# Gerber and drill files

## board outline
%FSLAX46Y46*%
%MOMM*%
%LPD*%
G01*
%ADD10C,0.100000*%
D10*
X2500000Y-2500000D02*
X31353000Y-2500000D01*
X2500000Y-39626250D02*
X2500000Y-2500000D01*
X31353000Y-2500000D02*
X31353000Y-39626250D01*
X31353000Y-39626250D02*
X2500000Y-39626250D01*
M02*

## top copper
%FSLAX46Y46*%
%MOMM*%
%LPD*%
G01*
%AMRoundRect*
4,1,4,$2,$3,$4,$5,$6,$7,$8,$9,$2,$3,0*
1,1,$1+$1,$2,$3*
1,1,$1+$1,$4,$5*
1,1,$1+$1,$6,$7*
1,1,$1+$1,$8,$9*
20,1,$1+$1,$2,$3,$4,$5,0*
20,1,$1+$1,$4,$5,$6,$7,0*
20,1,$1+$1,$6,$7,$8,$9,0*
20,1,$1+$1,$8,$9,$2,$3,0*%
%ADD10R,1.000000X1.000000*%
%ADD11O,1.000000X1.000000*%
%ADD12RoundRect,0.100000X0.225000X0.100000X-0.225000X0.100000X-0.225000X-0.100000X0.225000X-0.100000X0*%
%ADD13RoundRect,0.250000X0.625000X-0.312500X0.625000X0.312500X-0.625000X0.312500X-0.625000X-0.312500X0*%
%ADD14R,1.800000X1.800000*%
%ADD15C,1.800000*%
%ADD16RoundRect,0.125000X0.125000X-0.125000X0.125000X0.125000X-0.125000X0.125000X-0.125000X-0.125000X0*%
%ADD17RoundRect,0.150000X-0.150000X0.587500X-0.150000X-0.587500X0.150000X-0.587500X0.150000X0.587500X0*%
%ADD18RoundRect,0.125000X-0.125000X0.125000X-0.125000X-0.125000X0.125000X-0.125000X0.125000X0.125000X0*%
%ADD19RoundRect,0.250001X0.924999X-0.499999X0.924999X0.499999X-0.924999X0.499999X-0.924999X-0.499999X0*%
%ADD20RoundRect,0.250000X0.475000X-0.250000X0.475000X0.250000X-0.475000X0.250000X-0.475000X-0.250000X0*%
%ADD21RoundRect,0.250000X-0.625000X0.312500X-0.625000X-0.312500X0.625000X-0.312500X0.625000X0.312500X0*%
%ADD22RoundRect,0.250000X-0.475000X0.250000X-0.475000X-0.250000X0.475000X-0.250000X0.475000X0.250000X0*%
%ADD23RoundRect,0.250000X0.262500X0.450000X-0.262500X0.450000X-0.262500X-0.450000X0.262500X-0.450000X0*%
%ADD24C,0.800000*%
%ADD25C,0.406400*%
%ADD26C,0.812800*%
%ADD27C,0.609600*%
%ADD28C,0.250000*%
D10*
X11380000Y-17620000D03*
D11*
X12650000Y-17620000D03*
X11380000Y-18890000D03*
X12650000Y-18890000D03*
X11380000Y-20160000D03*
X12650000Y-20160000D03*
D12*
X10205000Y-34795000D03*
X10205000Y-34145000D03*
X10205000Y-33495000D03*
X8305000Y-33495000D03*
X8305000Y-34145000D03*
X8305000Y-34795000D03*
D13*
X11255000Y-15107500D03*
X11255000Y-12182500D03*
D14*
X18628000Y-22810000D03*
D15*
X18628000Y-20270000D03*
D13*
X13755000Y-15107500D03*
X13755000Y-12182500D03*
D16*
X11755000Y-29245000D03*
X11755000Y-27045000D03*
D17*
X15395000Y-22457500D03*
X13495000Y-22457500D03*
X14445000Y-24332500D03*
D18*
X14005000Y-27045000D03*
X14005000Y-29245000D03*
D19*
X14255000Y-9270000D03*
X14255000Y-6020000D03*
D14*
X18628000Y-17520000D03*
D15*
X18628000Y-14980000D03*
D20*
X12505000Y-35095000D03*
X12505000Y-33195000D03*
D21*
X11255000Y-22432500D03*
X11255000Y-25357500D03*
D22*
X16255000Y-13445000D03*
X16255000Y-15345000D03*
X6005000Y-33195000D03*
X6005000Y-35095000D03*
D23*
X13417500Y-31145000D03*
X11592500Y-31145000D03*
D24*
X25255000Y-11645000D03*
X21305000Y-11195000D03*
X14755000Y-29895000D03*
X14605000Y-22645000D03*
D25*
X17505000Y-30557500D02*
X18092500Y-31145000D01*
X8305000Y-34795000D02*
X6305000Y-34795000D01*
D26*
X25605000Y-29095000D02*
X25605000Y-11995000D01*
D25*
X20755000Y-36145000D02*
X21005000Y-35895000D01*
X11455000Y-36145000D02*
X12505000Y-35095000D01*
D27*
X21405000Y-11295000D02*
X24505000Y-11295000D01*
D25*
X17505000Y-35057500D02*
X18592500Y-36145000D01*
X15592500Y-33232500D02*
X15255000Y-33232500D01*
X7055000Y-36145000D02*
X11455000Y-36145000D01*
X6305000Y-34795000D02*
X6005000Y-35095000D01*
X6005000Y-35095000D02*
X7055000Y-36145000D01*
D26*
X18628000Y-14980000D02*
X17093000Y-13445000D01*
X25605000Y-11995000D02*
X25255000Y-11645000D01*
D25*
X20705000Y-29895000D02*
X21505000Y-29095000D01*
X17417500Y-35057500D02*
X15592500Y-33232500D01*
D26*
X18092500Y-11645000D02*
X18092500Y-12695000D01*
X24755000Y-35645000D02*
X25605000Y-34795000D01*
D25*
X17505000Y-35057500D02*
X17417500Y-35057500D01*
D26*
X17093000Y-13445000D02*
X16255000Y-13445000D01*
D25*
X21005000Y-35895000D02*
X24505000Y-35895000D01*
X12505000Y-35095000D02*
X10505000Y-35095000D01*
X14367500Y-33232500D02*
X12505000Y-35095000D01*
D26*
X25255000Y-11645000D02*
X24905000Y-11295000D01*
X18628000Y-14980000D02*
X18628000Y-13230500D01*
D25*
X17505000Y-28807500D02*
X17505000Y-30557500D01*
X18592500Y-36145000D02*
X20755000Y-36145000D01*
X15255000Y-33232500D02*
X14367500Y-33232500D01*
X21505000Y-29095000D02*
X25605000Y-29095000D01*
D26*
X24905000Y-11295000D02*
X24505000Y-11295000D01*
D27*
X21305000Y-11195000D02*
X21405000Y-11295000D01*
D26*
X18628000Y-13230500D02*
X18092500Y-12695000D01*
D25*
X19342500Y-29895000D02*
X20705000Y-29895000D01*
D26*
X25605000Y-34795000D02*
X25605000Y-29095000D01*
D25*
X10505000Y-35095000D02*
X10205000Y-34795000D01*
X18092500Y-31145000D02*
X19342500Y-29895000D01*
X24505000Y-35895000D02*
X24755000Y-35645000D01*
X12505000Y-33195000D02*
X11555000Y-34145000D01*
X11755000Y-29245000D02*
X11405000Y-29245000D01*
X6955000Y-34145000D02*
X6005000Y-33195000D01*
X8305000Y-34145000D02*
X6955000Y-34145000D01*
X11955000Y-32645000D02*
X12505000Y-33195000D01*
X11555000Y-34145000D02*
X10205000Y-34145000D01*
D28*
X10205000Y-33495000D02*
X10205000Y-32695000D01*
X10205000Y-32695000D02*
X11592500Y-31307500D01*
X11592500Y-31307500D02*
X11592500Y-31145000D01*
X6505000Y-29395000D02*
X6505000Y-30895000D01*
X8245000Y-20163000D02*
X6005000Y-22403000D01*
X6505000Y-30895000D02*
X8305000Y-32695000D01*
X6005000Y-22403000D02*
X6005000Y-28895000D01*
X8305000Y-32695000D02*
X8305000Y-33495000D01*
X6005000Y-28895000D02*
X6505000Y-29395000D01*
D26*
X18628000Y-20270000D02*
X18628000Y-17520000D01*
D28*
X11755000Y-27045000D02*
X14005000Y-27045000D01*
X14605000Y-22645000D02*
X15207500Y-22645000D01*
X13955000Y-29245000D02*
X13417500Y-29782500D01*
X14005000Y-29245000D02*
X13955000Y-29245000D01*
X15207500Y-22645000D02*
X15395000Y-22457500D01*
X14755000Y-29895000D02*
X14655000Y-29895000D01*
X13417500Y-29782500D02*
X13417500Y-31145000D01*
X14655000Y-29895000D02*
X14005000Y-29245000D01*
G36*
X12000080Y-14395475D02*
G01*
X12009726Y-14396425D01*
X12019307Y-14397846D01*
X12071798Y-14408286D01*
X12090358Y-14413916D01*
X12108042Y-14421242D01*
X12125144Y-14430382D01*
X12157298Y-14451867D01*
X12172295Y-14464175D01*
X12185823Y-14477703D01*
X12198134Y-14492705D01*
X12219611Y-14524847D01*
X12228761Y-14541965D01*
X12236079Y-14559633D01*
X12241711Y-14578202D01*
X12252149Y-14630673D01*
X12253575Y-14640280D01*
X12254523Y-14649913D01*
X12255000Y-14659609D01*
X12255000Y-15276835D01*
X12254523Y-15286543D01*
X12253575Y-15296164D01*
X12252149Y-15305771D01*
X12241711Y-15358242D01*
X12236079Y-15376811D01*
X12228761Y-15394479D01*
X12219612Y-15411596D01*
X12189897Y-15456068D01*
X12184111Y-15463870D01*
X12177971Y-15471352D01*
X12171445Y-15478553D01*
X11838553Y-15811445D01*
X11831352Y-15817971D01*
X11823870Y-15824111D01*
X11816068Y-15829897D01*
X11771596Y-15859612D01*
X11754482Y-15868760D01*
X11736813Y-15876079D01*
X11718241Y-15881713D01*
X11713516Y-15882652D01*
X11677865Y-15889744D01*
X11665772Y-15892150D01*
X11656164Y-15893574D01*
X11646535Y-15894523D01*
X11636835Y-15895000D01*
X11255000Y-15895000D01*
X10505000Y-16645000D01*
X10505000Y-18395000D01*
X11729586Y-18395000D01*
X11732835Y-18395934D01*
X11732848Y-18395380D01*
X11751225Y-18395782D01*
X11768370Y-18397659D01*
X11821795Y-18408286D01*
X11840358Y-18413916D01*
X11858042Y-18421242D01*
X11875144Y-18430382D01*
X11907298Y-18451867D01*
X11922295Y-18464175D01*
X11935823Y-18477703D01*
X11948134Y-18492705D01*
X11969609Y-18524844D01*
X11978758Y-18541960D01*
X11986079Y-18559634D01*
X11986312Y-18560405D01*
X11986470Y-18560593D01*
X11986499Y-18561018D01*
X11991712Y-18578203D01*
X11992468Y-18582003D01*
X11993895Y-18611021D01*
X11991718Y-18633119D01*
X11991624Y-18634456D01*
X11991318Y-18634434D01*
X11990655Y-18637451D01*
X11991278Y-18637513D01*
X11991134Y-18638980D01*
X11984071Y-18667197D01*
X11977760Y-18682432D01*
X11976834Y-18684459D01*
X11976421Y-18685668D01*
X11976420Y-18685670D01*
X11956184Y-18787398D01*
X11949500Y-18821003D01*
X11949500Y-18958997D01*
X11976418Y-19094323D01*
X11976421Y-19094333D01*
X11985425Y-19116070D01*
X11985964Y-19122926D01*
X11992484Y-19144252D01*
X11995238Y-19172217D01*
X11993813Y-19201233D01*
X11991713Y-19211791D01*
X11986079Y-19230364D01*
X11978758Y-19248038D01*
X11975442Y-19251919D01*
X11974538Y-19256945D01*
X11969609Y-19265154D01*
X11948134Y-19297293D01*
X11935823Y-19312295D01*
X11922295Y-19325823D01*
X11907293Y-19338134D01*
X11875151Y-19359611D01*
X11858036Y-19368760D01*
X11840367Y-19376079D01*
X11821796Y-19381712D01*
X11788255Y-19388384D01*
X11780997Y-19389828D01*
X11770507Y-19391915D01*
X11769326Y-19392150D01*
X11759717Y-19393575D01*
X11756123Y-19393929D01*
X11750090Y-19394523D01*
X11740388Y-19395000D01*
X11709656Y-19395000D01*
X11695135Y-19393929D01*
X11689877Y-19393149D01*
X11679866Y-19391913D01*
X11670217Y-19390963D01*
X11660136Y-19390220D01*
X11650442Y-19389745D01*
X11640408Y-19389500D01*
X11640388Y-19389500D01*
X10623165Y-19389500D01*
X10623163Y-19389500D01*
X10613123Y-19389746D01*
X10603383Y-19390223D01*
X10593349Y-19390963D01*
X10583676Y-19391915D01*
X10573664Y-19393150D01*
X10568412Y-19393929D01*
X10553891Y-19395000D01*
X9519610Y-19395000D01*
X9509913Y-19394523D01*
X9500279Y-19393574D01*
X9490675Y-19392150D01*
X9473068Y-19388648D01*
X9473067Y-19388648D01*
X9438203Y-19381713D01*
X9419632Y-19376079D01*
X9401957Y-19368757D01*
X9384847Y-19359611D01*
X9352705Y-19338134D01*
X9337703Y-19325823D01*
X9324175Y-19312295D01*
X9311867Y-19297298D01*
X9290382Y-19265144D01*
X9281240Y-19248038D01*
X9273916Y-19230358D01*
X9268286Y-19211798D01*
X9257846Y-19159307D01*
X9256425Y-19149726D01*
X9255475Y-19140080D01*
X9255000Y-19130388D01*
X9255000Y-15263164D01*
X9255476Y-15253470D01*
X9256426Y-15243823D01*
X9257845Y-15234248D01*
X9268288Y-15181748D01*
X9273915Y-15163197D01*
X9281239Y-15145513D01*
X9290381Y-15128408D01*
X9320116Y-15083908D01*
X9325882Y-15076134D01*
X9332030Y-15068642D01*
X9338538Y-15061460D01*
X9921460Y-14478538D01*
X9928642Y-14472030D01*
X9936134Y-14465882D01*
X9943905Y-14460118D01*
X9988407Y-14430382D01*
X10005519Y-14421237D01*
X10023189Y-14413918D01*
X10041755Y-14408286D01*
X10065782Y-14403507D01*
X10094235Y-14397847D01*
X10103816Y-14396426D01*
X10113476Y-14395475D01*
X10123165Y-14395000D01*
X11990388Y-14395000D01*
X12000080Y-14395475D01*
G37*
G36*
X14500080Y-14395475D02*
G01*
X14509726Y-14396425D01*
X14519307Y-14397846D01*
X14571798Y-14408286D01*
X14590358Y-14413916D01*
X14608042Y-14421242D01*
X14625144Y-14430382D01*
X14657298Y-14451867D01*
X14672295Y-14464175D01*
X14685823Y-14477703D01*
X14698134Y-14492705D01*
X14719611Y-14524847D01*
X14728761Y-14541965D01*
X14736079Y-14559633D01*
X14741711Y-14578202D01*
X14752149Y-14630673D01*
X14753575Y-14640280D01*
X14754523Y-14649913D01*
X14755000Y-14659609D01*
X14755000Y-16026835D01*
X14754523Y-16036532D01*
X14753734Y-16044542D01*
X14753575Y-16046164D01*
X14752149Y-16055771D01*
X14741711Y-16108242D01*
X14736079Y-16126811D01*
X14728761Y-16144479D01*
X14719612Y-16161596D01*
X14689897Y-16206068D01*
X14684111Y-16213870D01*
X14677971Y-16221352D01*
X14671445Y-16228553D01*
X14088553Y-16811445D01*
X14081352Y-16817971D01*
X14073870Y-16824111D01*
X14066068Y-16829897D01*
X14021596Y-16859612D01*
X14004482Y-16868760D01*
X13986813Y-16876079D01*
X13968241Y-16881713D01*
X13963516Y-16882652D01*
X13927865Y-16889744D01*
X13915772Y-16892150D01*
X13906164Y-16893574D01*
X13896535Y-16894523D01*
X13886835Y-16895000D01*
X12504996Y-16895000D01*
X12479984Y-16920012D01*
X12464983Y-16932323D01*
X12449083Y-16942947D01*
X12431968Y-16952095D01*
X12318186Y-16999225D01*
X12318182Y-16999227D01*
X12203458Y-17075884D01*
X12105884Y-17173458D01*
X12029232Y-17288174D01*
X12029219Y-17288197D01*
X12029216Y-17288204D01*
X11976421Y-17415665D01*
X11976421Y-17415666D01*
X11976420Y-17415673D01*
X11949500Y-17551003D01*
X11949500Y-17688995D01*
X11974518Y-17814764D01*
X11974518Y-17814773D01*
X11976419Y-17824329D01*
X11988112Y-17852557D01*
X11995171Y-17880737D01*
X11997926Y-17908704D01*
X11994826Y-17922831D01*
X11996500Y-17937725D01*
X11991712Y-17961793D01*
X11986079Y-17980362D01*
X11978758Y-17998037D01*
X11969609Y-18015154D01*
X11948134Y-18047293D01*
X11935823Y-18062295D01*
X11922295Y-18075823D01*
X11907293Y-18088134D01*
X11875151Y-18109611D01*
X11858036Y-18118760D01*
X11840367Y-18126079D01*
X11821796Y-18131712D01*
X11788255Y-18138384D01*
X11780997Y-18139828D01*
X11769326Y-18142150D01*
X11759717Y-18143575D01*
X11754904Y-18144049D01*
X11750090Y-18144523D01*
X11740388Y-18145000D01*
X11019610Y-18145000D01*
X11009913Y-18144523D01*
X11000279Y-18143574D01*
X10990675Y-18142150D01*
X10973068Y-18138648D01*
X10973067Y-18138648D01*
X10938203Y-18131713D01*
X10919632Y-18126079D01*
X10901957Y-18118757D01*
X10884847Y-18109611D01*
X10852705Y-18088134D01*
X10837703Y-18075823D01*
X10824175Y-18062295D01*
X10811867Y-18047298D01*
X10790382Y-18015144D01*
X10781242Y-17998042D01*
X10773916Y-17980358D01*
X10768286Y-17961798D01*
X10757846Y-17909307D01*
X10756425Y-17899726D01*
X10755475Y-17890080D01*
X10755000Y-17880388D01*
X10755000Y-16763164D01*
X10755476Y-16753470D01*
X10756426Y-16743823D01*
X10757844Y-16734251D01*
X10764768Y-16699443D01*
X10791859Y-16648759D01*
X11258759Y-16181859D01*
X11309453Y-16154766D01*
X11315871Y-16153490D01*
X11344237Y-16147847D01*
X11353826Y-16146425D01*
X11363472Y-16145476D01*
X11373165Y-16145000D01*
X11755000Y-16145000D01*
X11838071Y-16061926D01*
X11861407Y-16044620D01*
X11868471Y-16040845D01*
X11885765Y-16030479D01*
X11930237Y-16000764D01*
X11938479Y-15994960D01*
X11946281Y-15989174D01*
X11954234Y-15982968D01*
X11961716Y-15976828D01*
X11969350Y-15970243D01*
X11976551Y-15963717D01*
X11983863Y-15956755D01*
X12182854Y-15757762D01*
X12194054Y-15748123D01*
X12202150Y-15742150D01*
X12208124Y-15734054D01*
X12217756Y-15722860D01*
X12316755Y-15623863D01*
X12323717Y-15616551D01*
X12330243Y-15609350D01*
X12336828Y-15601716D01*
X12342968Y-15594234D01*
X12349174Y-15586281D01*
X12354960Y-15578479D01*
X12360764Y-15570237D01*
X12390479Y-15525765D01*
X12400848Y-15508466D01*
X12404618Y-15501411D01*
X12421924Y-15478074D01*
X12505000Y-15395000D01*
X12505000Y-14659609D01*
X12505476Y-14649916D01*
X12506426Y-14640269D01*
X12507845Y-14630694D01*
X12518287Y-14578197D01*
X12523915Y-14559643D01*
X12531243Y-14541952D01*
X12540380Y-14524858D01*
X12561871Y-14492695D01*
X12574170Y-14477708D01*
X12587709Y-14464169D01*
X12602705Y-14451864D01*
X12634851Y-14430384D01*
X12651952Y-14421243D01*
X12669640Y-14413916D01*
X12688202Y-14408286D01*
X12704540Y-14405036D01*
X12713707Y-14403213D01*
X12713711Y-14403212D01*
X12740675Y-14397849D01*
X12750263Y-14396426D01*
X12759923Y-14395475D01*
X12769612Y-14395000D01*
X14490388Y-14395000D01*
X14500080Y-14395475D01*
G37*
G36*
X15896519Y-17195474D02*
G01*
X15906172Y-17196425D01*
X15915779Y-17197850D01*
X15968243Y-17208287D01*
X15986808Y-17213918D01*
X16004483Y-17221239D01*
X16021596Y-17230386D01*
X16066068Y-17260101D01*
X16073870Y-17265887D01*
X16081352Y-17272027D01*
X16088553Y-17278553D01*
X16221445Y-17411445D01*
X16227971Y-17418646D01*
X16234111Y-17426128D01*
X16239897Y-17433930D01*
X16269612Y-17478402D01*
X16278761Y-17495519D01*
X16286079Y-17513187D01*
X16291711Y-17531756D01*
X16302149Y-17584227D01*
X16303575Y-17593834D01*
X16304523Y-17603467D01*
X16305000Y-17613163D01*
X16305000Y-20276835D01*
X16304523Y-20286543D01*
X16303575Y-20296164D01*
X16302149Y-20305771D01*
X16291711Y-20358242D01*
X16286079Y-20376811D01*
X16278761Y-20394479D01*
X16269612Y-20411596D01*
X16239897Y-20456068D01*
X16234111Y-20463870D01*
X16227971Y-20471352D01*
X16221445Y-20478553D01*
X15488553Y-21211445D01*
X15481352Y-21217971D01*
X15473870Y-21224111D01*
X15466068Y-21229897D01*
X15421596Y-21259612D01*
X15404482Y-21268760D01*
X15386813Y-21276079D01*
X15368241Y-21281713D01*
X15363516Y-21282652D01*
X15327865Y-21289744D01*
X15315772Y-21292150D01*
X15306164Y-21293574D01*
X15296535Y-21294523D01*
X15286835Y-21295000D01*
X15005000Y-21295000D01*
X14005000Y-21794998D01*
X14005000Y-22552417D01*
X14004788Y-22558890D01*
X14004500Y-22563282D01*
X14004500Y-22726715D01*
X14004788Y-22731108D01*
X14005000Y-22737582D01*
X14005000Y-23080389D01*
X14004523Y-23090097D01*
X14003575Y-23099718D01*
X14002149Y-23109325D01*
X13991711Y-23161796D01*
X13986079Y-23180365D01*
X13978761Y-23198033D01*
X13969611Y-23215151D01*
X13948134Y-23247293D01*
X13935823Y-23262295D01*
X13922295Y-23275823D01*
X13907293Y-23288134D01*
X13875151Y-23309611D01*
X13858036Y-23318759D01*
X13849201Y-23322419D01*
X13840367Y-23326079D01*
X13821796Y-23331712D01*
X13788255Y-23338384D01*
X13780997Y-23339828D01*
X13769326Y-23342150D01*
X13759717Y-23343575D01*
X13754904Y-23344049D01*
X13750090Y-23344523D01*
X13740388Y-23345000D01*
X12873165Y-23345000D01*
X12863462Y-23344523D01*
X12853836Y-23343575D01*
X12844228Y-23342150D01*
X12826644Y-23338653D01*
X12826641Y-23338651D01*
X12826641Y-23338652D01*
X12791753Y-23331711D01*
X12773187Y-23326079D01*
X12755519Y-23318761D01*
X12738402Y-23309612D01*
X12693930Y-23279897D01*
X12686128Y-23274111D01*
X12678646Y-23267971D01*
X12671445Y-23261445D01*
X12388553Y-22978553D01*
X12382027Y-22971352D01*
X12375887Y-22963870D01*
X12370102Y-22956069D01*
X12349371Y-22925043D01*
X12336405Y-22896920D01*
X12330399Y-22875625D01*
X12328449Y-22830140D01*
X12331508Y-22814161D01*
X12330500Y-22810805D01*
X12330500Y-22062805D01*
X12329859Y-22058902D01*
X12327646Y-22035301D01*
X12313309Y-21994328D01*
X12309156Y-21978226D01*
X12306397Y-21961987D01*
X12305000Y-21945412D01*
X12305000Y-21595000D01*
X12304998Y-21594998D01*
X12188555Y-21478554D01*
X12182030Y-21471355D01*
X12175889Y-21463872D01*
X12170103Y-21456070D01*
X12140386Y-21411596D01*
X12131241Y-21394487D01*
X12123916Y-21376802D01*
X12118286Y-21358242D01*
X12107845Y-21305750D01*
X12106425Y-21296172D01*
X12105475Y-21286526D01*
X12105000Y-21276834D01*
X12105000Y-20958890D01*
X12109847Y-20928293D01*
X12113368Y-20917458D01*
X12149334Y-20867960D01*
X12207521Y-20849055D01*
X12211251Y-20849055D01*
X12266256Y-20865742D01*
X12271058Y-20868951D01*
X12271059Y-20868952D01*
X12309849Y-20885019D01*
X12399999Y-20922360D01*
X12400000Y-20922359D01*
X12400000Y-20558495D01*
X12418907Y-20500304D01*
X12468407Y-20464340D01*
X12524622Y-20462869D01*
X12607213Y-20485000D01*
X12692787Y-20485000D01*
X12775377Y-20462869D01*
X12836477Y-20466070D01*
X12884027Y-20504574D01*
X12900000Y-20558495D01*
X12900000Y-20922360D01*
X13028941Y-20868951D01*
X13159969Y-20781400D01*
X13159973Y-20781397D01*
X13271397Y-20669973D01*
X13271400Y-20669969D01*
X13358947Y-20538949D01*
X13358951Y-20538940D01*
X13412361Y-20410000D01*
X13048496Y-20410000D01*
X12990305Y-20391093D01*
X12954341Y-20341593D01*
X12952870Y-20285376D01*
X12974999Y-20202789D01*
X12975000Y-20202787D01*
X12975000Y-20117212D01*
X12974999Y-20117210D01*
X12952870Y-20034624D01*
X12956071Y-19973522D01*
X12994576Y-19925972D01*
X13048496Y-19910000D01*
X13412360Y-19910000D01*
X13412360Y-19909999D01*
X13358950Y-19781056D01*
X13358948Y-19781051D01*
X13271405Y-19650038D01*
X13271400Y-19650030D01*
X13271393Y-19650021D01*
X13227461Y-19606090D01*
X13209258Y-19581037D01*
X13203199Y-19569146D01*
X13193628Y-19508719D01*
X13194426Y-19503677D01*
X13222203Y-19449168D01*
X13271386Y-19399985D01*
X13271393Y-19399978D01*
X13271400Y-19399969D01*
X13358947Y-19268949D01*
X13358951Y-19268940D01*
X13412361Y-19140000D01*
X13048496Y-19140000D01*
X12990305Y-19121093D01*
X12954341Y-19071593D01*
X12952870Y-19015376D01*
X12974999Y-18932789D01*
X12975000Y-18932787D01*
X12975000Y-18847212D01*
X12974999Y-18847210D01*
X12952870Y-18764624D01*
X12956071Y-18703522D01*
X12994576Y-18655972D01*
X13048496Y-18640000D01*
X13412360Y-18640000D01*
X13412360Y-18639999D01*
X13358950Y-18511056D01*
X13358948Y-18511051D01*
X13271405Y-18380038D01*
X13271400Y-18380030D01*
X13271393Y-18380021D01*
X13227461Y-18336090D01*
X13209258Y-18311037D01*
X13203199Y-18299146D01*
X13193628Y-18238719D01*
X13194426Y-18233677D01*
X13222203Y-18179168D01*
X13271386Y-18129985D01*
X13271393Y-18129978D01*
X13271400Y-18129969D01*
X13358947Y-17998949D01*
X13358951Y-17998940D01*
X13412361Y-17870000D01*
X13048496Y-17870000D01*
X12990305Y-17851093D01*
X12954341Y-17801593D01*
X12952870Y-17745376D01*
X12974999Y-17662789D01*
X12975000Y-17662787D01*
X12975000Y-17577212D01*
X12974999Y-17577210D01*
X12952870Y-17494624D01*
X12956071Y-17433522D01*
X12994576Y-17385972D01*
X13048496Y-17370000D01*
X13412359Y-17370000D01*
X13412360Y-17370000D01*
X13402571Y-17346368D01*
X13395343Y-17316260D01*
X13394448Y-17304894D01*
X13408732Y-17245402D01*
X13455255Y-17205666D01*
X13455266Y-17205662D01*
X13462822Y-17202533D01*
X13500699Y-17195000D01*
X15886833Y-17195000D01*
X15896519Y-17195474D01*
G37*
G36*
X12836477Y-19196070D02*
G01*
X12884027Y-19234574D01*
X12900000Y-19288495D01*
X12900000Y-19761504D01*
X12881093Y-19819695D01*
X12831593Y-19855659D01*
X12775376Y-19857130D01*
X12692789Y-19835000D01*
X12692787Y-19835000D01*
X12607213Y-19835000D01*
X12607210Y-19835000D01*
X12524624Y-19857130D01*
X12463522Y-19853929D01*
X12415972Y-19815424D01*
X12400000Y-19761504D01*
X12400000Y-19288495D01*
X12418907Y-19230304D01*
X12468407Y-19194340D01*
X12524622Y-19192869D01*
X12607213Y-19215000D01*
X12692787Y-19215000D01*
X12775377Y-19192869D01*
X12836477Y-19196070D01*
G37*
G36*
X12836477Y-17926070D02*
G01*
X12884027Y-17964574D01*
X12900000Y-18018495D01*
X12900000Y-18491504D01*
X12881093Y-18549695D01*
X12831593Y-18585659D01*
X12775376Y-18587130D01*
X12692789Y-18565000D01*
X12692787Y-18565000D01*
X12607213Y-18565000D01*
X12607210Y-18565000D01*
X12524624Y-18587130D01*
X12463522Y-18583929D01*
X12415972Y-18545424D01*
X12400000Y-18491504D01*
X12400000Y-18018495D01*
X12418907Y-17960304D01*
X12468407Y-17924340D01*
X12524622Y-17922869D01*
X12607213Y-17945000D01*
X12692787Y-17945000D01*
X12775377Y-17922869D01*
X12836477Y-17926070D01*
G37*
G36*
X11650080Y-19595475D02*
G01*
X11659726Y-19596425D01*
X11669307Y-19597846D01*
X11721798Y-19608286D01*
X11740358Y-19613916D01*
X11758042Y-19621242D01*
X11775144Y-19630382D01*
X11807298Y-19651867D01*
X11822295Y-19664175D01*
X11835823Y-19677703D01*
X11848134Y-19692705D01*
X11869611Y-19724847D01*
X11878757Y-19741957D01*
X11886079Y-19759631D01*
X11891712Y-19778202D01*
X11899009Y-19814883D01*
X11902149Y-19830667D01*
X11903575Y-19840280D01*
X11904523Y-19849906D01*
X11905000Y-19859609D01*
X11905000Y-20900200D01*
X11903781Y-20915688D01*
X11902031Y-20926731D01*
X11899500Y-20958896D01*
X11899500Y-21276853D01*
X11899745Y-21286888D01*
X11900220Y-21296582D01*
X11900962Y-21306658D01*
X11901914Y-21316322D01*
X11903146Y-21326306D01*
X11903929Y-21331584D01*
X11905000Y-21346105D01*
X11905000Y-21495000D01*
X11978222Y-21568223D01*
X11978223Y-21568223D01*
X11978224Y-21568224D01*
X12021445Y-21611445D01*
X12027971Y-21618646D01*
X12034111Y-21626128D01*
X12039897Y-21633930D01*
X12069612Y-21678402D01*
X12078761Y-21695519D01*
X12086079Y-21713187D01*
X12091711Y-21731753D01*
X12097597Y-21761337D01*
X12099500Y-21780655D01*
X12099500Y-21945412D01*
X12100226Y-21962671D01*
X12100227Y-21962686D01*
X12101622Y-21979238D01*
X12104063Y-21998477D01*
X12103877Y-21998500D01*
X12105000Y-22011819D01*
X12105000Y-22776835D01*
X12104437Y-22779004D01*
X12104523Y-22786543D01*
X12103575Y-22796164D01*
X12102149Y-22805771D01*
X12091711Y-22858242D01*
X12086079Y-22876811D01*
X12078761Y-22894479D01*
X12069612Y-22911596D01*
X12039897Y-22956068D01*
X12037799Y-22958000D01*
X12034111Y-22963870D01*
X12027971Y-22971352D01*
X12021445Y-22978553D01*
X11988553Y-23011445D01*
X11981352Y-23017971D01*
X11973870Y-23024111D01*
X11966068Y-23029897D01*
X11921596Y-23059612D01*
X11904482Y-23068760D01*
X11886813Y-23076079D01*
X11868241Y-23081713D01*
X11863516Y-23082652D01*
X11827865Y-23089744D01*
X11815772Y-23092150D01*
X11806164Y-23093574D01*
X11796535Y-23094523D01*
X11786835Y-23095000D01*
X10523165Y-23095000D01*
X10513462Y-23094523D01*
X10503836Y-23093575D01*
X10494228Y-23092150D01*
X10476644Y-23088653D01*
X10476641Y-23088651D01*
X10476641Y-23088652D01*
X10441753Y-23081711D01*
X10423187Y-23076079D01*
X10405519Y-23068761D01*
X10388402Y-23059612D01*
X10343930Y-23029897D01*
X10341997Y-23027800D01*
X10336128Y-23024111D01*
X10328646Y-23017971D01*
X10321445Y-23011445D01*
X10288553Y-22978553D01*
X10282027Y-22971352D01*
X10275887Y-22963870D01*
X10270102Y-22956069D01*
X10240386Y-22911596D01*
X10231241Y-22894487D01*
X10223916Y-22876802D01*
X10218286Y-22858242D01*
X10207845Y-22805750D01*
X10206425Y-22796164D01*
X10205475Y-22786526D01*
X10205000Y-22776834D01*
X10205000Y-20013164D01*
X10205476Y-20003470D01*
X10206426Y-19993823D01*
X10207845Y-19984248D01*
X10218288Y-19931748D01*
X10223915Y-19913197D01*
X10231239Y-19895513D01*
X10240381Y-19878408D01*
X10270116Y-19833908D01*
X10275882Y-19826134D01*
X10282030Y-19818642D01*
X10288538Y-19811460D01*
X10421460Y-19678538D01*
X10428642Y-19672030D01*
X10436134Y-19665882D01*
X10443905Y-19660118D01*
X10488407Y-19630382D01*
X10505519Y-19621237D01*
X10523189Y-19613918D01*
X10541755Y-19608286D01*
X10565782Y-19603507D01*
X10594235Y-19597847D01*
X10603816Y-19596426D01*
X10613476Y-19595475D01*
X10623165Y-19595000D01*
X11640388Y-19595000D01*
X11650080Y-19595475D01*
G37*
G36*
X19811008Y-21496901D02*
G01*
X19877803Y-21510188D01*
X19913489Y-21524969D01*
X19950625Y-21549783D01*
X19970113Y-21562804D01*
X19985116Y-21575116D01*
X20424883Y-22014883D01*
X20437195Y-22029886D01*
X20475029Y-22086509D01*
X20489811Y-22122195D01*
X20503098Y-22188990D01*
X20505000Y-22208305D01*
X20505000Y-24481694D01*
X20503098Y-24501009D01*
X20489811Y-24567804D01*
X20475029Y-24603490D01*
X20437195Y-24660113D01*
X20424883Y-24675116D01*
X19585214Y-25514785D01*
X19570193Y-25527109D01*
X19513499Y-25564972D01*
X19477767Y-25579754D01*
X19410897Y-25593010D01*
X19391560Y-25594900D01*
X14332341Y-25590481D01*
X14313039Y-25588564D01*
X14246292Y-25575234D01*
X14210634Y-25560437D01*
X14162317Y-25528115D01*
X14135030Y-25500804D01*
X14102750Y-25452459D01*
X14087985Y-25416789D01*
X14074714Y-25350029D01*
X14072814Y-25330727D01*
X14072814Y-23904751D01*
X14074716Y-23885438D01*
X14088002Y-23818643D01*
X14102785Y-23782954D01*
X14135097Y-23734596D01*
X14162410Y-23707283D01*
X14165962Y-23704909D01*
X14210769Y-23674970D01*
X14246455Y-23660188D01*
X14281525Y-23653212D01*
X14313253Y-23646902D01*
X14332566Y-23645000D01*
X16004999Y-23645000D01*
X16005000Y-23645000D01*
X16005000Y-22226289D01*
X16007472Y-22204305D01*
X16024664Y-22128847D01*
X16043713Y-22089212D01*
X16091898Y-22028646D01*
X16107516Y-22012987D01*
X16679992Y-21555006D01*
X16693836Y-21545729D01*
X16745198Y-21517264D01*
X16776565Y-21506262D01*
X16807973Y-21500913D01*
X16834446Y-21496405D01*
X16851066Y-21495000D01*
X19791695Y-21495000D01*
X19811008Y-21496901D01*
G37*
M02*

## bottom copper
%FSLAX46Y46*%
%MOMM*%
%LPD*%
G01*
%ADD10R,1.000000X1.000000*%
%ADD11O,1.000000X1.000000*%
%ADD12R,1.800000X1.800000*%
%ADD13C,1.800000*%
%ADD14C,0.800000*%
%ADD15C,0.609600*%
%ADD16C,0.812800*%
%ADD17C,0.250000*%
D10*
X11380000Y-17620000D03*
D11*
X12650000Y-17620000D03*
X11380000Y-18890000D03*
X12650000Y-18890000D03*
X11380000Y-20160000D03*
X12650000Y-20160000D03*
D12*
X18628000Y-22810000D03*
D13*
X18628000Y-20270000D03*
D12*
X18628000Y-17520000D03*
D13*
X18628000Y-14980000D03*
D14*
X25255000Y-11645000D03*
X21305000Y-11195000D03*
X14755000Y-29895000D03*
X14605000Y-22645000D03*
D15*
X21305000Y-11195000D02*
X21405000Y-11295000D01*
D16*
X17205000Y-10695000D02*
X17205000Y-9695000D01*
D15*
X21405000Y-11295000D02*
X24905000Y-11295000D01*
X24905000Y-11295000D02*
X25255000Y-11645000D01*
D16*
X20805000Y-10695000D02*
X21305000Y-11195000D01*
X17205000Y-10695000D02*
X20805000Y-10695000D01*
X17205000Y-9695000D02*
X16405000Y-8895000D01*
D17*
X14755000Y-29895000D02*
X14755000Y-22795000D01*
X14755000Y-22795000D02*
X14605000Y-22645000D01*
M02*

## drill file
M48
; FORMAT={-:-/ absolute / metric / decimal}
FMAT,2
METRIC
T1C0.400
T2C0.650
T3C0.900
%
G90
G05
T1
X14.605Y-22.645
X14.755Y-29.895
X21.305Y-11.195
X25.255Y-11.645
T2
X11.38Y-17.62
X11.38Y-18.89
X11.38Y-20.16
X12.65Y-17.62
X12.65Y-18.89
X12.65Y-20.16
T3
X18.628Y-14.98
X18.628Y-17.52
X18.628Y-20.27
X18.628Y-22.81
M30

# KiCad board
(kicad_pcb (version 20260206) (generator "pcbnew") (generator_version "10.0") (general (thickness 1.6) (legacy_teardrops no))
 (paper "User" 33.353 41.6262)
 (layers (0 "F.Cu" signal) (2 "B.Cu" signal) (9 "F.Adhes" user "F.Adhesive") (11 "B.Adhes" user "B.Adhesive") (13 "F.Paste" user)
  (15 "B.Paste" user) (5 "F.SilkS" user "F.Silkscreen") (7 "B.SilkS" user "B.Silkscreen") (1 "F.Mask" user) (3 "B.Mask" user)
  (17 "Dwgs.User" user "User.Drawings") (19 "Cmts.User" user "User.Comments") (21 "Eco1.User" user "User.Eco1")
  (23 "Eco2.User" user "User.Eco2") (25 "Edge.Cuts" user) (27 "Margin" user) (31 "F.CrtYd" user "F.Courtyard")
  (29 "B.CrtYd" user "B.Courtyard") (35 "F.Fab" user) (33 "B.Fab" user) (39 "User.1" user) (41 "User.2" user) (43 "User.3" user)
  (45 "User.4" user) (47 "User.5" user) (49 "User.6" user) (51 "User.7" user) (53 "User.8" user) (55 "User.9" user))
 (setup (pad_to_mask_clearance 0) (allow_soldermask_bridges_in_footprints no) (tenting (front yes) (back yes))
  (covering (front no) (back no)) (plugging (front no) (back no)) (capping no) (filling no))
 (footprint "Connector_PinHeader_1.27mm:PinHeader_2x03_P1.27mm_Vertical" (layer "F.Cu") (at 11.38 17.62)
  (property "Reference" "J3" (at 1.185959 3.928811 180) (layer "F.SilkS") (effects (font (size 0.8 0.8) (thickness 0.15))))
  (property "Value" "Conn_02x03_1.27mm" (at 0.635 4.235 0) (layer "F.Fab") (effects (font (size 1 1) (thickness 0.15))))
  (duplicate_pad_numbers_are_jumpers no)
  (pad "1" thru_hole rect (at 0 0) (size 1 1) (drill 0.65) (layers "*.Cu" "*.Mask") (remove_unused_layers no) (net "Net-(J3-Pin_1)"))
  (pad "2" thru_hole oval (at 1.27 0) (size 1 1) (drill 0.65) (layers "*.Cu" "*.Mask") (remove_unused_layers no) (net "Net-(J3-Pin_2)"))
  (pad "3" thru_hole oval (at 0 1.27) (size 1 1) (drill 0.65) (layers "*.Cu" "*.Mask") (remove_unused_layers no) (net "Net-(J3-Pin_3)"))
  (pad "4" thru_hole oval (at 1.27 1.27) (size 1 1) (drill 0.65) (layers "*.Cu" "*.Mask") (remove_unused_layers no) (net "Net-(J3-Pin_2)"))
  (pad "5" thru_hole oval (at 0 2.54) (size 1 1) (drill 0.65) (layers "*.Cu" "*.Mask") (remove_unused_layers no) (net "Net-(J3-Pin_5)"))
  (pad "6" thru_hole oval (at 1.27 2.54) (size 1 1) (drill 0.65) (layers "*.Cu" "*.Mask") (remove_unused_layers no) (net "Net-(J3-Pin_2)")))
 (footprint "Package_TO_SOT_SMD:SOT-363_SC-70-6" (layer "F.Cu") (at 9.255 34.145 180)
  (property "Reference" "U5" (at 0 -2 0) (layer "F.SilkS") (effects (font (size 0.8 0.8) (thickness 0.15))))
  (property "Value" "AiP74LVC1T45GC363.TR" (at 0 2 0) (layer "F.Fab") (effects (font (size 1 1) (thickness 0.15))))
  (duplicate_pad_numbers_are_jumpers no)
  (pad "1" smd roundrect (at -0.95 -0.65 180) (size 0.65 0.4) (layers "F.Cu" "F.Mask" "F.Paste") (roundrect_rratio 0.25) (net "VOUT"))
  (pad "2" smd roundrect (at -0.95 0 180) (size 0.65 0.4) (layers "F.Cu" "F.Mask" "F.Paste") (roundrect_rratio 0.25) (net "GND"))
  (pad "3" smd roundrect (at -0.95 0.65 180) (size 0.65 0.4) (layers "F.Cu" "F.Mask" "F.Paste") (roundrect_rratio 0.25) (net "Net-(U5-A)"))
  (pad "4" smd roundrect (at 0.95 0.65 180) (size 0.65 0.4) (layers "F.Cu" "F.Mask" "F.Paste") (roundrect_rratio 0.25) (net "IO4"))
  (pad "5" smd roundrect (at 0.95 0 180) (size 0.65 0.4) (layers "F.Cu" "F.Mask" "F.Paste") (roundrect_rratio 0.25) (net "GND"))
  (pad "6" smd roundrect (at 0.95 -0.65 180) (size 0.65 0.4) (layers "F.Cu" "F.Mask" "F.Paste") (roundrect_rratio 0.25) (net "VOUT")))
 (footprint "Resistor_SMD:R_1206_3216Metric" (layer "F.Cu") (at 11.255 13.645 90)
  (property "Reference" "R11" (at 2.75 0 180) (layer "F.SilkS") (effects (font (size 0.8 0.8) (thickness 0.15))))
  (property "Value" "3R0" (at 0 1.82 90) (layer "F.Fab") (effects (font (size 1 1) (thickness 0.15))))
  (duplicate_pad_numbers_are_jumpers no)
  (pad "1" smd roundrect (at -1.4625 0 90) (size 1.125 1.75) (layers "F.Cu" "F.Mask" "F.Paste") (roundrect_rratio 0.2222222222)
   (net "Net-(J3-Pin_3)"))
  (pad "2" smd roundrect (at 1.4625 0 90) (size 1.125 1.75) (layers "F.Cu" "F.Mask" "F.Paste") (roundrect_rratio 0.2222222222) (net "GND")))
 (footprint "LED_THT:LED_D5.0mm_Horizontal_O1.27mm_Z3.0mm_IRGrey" (layer "F.Cu") (at 18.628 22.81 90)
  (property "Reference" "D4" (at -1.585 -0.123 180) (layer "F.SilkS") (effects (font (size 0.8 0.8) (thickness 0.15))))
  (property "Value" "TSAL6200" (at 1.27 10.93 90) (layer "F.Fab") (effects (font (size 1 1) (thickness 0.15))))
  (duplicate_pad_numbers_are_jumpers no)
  (pad "1" thru_hole rect (at 0 0 90) (size 1.8 1.8) (drill 0.9) (layers "*.Cu" "*.Mask") (remove_unused_layers no) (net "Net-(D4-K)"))
  (pad "2" thru_hole circle (at 2.54 0 90) (size 1.8 1.8) (drill 0.9) (layers "*.Cu" "*.Mask") (remove_unused_layers no) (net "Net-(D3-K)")))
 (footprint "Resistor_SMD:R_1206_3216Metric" (layer "F.Cu") (at 13.755 13.645 90)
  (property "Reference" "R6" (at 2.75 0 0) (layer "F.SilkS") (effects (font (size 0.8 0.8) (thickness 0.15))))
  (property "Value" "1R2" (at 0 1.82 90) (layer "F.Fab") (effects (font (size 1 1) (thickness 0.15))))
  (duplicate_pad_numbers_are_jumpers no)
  (pad "1" smd roundrect (at -1.4625 0 90) (size 1.125 1.75) (layers "F.Cu" "F.Mask" "F.Paste") (roundrect_rratio 0.2222222222)
   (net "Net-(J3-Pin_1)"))
  (pad "2" smd roundrect (at 1.4625 0 90) (size 1.125 1.75) (layers "F.Cu" "F.Mask" "F.Paste") (roundrect_rratio 0.2222222222) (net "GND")))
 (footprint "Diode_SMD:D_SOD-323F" (layer "F.Cu") (at 11.755 28.145 90)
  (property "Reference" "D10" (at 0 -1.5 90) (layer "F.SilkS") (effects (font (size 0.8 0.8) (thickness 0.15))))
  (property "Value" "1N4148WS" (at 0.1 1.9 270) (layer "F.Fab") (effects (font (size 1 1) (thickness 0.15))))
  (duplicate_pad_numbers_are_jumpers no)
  (pad "1" smd roundrect (at -1.1 0 90) (size 0.5 0.5) (layers "F.Cu" "F.Mask" "F.Paste") (roundrect_rratio 0.25) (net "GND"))
  (pad "2" smd roundrect (at 1.1 0 90) (size 0.5 0.5) (layers "F.Cu" "F.Mask" "F.Paste") (roundrect_rratio 0.25) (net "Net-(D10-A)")))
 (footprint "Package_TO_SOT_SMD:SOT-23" (layer "F.Cu") (at 14.445 23.395 -90)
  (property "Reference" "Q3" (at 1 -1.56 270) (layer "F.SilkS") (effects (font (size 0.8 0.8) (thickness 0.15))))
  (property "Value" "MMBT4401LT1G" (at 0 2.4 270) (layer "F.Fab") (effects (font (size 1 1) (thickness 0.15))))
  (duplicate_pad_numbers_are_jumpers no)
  (pad "1" smd roundrect (at -0.9375 -0.95 270) (size 1.475 0.6) (layers "F.Cu" "F.Mask" "F.Paste") (roundrect_rratio 0.25)
   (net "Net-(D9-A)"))
  (pad "2" smd roundrect (at -0.9375 0.95 270) (size 1.475 0.6) (layers "F.Cu" "F.Mask" "F.Paste") (roundrect_rratio 0.25)
   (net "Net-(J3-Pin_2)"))
  (pad "3" smd roundrect (at 0.9375 0 270) (size 1.475 0.6) (layers "F.Cu" "F.Mask" "F.Paste") (roundrect_rratio 0.25) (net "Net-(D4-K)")))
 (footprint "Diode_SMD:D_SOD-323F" (layer "F.Cu") (at 14.005 28.145 -90)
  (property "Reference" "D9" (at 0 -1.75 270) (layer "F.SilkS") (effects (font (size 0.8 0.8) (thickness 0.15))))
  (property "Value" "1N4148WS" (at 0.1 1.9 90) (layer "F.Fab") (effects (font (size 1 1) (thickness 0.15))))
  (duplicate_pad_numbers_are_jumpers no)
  (pad "1" smd roundrect (at -1.1 0 270) (size 0.5 0.5) (layers "F.Cu" "F.Mask" "F.Paste") (roundrect_rratio 0.25) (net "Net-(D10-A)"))
  (pad "2" smd roundrect (at 1.1 0 270) (size 0.5 0.5) (layers "F.Cu" "F.Mask" "F.Paste") (roundrect_rratio 0.25) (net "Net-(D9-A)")))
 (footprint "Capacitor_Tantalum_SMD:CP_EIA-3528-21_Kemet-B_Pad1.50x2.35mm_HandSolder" (layer "F.Cu") (at 14.255 7.645 90)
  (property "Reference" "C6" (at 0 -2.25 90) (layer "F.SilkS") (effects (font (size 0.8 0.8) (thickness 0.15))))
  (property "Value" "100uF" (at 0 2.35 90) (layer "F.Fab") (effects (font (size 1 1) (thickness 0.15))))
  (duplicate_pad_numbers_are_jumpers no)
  (pad "1" smd roundrect (at -1.625 0 90) (size 1.5 2.35) (layers "F.Cu" "F.Mask" "F.Paste") (roundrect_rratio 0.1666673333) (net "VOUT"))
  (pad "2" smd roundrect (at 1.625 0 90) (size 1.5 2.35) (layers "F.Cu" "F.Mask" "F.Paste") (roundrect_rratio 0.1666673333) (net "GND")))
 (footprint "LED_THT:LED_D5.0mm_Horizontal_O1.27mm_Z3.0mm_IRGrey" (layer "F.Cu") (at 18.628 17.52 90)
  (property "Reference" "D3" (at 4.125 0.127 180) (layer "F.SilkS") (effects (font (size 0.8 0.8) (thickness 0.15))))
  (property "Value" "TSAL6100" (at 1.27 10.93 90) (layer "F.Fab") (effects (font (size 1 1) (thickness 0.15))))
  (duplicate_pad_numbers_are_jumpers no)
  (pad "1" thru_hole rect (at 0 0 90) (size 1.8 1.8) (drill 0.9) (layers "*.Cu" "*.Mask") (remove_unused_layers no) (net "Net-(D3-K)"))
  (pad "2" thru_hole circle (at 2.54 0 90) (size 1.8 1.8) (drill 0.9) (layers "*.Cu" "*.Mask") (remove_unused_layers no) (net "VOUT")))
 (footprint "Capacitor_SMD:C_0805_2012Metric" (layer "F.Cu") (at 12.505 34.145 90)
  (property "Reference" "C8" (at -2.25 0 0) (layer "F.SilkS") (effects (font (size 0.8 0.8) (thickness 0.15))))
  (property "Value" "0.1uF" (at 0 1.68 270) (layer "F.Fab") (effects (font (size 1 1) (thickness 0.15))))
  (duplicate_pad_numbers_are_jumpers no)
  (pad "1" smd roundrect (at -0.95 0 90) (size 1 1.45) (layers "F.Cu" "F.Mask" "F.Paste") (roundrect_rratio 0.25) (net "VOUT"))
  (pad "2" smd roundrect (at 0.95 0 90) (size 1 1.45) (layers "F.Cu" "F.Mask" "F.Paste") (roundrect_rratio 0.25) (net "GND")))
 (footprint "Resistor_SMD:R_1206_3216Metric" (layer "F.Cu") (at 11.255 23.895 -90)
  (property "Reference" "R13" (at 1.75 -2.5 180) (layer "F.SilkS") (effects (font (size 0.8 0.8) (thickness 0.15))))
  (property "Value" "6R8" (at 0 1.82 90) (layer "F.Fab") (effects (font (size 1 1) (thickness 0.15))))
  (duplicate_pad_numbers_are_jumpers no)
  (pad "1" smd roundrect (at -1.4625 0 270) (size 1.125 1.75) (layers "F.Cu" "F.Mask" "F.Paste") (roundrect_rratio 0.2222222222)
   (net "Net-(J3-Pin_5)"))
  (pad "2" smd roundrect (at 1.4625 0 270) (size 1.125 1.75) (layers "F.Cu" "F.Mask" "F.Paste") (roundrect_rratio 0.2222222222) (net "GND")))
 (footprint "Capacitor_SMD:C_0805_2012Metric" (layer "F.Cu") (at 16.255 14.395 -90)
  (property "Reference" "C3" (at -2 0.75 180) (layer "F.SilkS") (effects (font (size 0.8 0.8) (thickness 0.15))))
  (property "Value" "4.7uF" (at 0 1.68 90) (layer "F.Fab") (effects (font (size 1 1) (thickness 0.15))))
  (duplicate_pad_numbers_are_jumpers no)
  (pad "1" smd roundrect (at -0.95 0 270) (size 1 1.45) (layers "F.Cu" "F.Mask" "F.Paste") (roundrect_rratio 0.25) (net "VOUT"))
  (pad "2" smd roundrect (at 0.95 0 270) (size 1 1.45) (layers "F.Cu" "F.Mask" "F.Paste") (roundrect_rratio 0.25) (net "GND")))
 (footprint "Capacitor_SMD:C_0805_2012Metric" (layer "F.Cu") (at 6.005 34.145 -90)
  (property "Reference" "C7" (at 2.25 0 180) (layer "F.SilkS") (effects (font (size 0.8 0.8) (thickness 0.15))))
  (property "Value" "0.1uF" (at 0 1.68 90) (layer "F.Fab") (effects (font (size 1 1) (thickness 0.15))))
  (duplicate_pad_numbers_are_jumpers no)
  (pad "1" smd roundrect (at -0.95 0 270) (size 1 1.45) (layers "F.Cu" "F.Mask" "F.Paste") (roundrect_rratio 0.25) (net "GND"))
  (pad "2" smd roundrect (at 0.95 0 270) (size 1 1.45) (layers "F.Cu" "F.Mask" "F.Paste") (roundrect_rratio 0.25) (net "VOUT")))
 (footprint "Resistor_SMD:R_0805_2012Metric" (layer "F.Cu") (at 12.505 31.145 180)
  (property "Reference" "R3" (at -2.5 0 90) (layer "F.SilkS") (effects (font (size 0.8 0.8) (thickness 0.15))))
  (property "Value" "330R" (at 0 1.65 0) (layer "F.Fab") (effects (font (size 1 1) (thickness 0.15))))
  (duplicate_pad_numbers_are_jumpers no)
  (pad "1" smd roundrect (at -0.9125 0 180) (size 1.025 1.4) (layers "F.Cu" "F.Mask" "F.Paste") (roundrect_rratio 0.243902439)
   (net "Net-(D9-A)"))
  (pad "2" smd roundrect (at 0.9125 0 180) (size 1.025 1.4) (layers "F.Cu" "F.Mask" "F.Paste") (roundrect_rratio 0.243902439)
   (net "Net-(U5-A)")))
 (gr_line (start 2.5 2.5) (end 31.353 2.5) (stroke (width 0.1) (type default)) (layer "Edge.Cuts"))
 (gr_line (start 2.5 39.62625) (end 2.5 2.5) (stroke (width 0.1) (type default)) (layer "Edge.Cuts"))
 (gr_line (start 31.353 2.5) (end 31.353 39.62625) (stroke (width 0.1) (type default)) (layer "Edge.Cuts"))
 (gr_line (start 31.353 39.62625) (end 2.5 39.62625) (stroke (width 0.1) (type default)) (layer "Edge.Cuts"))
 (segment (start 17.505 30.5575) (end 18.0925 31.145) (width 0.4064) (layer "F.Cu") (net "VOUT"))
 (segment (start 8.305 34.795) (end 6.305 34.795) (width 0.4064) (layer "F.Cu") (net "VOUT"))
 (segment (start 25.605 29.095) (end 25.605 11.995) (width 0.8128) (layer "F.Cu") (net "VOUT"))
 (segment (start 20.755 36.145) (end 21.005 35.895) (width 0.4064) (layer "F.Cu") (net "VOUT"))
 (segment (start 11.455 36.145) (end 12.505 35.095) (width 0.4064) (layer "F.Cu") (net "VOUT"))
 (segment (start 21.405 11.295) (end 24.505 11.295) (width 0.6096) (layer "F.Cu") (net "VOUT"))
 (segment (start 17.505 35.0575) (end 18.5925 36.145) (width 0.4064) (layer "F.Cu") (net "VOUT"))
 (segment (start 15.5925 33.2325) (end 15.255 33.2325) (width 0.4064) (layer "F.Cu") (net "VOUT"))
 (segment (start 7.055 36.145) (end 11.455 36.145) (width 0.4064) (layer "F.Cu") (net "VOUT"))
 (segment (start 6.305 34.795) (end 6.005 35.095) (width 0.4064) (layer "F.Cu") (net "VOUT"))
 (segment (start 6.005 35.095) (end 7.055 36.145) (width 0.4064) (layer "F.Cu") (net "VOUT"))
 (segment (start 18.628 14.98) (end 17.093 13.445) (width 0.8128) (layer "F.Cu") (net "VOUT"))
 (segment (start 25.605 11.995) (end 25.255 11.645) (width 0.8128) (layer "F.Cu") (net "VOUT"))
 (segment (start 20.705 29.895) (end 21.505 29.095) (width 0.4064) (layer "F.Cu") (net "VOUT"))
 (segment (start 17.4175 35.0575) (end 15.5925 33.2325) (width 0.4064) (layer "F.Cu") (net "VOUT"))
 (segment (start 18.0925 11.645) (end 18.0925 12.695) (width 0.8128) (layer "F.Cu") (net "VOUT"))
 (segment (start 24.755 35.645) (end 25.605 34.795) (width 0.8128) (layer "F.Cu") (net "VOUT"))
 (segment (start 17.505 35.0575) (end 17.4175 35.0575) (width 0.4064) (layer "F.Cu") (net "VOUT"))
 (segment (start 17.093 13.445) (end 16.255 13.445) (width 0.8128) (layer "F.Cu") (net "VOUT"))
 (segment (start 21.005 35.895) (end 24.505 35.895) (width 0.4064) (layer "F.Cu") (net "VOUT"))
 (segment (start 12.505 35.095) (end 10.505 35.095) (width 0.4064) (layer "F.Cu") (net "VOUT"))
 (segment (start 14.3675 33.2325) (end 12.505 35.095) (width 0.4064) (layer "F.Cu") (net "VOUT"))
 (segment (start 25.255 11.645) (end 24.905 11.295) (width 0.8128) (layer "F.Cu") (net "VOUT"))
 (segment (start 18.628 14.98) (end 18.628 13.2305) (width 0.8128) (layer "F.Cu") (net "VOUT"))
 (segment (start 17.505 28.8075) (end 17.505 30.5575) (width 0.4064) (layer "F.Cu") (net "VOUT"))
 (segment (start 18.5925 36.145) (end 20.755 36.145) (width 0.4064) (layer "F.Cu") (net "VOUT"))
 (segment (start 15.255 33.2325) (end 14.3675 33.2325) (width 0.4064) (layer "F.Cu") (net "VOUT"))
 (segment (start 21.505 29.095) (end 25.605 29.095) (width 0.4064) (layer "F.Cu") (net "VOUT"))
 (segment (start 24.905 11.295) (end 24.505 11.295) (width 0.8128) (layer "F.Cu") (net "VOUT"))
 (segment (start 21.305 11.195) (end 21.405 11.295) (width 0.6096) (layer "F.Cu") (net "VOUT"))
 (segment (start 18.628 13.2305) (end 18.0925 12.695) (width 0.8128) (layer "F.Cu") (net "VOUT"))
 (segment (start 19.3425 29.895) (end 20.705 29.895) (width 0.4064) (layer "F.Cu") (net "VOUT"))
 (segment (start 25.605 34.795) (end 25.605 29.095) (width 0.8128) (layer "F.Cu") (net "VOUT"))
 (segment (start 10.505 35.095) (end 10.205 34.795) (width 0.4064) (layer "F.Cu") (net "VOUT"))
 (segment (start 18.0925 31.145) (end 19.3425 29.895) (width 0.4064) (layer "F.Cu") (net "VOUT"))
 (segment (start 24.505 35.895) (end 24.755 35.645) (width 0.4064) (layer "F.Cu") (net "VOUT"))
 (via (at 25.255 11.645) (size 0.8) (drill 0.4) (layers "F.Cu" "B.Cu") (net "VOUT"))
 (via (at 21.305 11.195) (size 0.8) (drill 0.4) (layers "F.Cu" "B.Cu") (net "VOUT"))
 (segment (start 21.305 11.195) (end 21.405 11.295) (width 0.6096) (layer "B.Cu") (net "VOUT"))
 (segment (start 17.205 10.695) (end 17.205 9.695) (width 0.8128) (layer "B.Cu") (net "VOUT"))
 (segment (start 21.405 11.295) (end 24.905 11.295) (width 0.6096) (layer "B.Cu") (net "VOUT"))
 (segment (start 24.905 11.295) (end 25.255 11.645) (width 0.6096) (layer "B.Cu") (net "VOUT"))
 (segment (start 20.805 10.695) (end 21.305 11.195) (width 0.8128) (layer "B.Cu") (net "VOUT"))
 (segment (start 17.205 10.695) (end 20.805 10.695) (width 0.8128) (layer "B.Cu") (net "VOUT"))
 (segment (start 17.205 9.695) (end 16.405 8.895) (width 0.8128) (layer "B.Cu") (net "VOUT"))
 (segment (start 12.505 33.195) (end 11.555 34.145) (width 0.4064) (layer "F.Cu") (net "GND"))
 (segment (start 11.755 29.245) (end 11.405 29.245) (width 0.4064) (layer "F.Cu") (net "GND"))
 (segment (start 6.955 34.145) (end 6.005 33.195) (width 0.4064) (layer "F.Cu") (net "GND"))
 (segment (start 8.305 34.145) (end 6.955 34.145) (width 0.4064) (layer "F.Cu") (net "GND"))
 (segment (start 11.955 32.645) (end 12.505 33.195) (width 0.4064) (layer "F.Cu") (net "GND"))
 (segment (start 11.555 34.145) (end 10.205 34.145) (width 0.4064) (layer "F.Cu") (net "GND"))
 (segment (start 10.205 33.495) (end 10.205 32.695) (width 0.25) (layer "F.Cu") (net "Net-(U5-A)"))
 (segment (start 10.205 32.695) (end 11.5925 31.3075) (width 0.25) (layer "F.Cu") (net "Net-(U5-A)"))
 (segment (start 11.5925 31.3075) (end 11.5925 31.145) (width 0.25) (layer "F.Cu") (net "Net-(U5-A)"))
 (segment (start 6.505 29.395) (end 6.505 30.895) (width 0.25) (layer "F.Cu") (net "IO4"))
 (segment (start 8.245 20.163) (end 6.005 22.403) (width 0.25) (layer "F.Cu") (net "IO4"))
 (segment (start 6.505 30.895) (end 8.305 32.695) (width 0.25) (layer "F.Cu") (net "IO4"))
 (segment (start 6.005 22.403) (end 6.005 28.895) (width 0.25) (layer "F.Cu") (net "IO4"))
 (segment (start 8.305 32.695) (end 8.305 33.495) (width 0.25) (layer "F.Cu") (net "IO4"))
 (segment (start 6.005 28.895) (end 6.505 29.395) (width 0.25) (layer "F.Cu") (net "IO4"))
 (segment (start 18.628 20.27) (end 18.628 17.52) (width 0.8128) (layer "F.Cu") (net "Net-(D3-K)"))
 (segment (start 11.755 27.045) (end 14.005 27.045) (width 0.25) (layer "F.Cu") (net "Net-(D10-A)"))
 (segment (start 14.605 22.645) (end 15.2075 22.645) (width 0.25) (layer "F.Cu") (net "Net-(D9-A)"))
 (segment (start 13.955 29.245) (end 13.4175 29.7825) (width 0.25) (layer "F.Cu") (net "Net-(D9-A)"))
 (segment (start 14.005 29.245) (end 13.955 29.245) (width 0.25) (layer "F.Cu") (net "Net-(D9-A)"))
 (segment (start 15.2075 22.645) (end 15.395 22.4575) (width 0.25) (layer "F.Cu") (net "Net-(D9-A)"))
 (segment (start 14.755 29.895) (end 14.655 29.895) (width 0.25) (layer "F.Cu") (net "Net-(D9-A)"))
 (segment (start 13.4175 29.7825) (end 13.4175 31.145) (width 0.25) (layer "F.Cu") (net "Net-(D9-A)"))
 (segment (start 14.655 29.895) (end 14.005 29.245) (width 0.25) (layer "F.Cu") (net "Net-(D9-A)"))
 (via (at 14.755 29.895) (size 0.8) (drill 0.4) (layers "F.Cu" "B.Cu") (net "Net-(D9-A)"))
 (via (at 14.605 22.645) (size 0.8) (drill 0.4) (layers "F.Cu" "B.Cu") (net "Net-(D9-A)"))
 (segment (start 14.755 29.895) (end 14.755 22.795) (width 0.25) (layer "B.Cu") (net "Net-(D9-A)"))
 (segment (start 14.755 22.795) (end 14.605 22.645) (width 0.25) (layer "B.Cu") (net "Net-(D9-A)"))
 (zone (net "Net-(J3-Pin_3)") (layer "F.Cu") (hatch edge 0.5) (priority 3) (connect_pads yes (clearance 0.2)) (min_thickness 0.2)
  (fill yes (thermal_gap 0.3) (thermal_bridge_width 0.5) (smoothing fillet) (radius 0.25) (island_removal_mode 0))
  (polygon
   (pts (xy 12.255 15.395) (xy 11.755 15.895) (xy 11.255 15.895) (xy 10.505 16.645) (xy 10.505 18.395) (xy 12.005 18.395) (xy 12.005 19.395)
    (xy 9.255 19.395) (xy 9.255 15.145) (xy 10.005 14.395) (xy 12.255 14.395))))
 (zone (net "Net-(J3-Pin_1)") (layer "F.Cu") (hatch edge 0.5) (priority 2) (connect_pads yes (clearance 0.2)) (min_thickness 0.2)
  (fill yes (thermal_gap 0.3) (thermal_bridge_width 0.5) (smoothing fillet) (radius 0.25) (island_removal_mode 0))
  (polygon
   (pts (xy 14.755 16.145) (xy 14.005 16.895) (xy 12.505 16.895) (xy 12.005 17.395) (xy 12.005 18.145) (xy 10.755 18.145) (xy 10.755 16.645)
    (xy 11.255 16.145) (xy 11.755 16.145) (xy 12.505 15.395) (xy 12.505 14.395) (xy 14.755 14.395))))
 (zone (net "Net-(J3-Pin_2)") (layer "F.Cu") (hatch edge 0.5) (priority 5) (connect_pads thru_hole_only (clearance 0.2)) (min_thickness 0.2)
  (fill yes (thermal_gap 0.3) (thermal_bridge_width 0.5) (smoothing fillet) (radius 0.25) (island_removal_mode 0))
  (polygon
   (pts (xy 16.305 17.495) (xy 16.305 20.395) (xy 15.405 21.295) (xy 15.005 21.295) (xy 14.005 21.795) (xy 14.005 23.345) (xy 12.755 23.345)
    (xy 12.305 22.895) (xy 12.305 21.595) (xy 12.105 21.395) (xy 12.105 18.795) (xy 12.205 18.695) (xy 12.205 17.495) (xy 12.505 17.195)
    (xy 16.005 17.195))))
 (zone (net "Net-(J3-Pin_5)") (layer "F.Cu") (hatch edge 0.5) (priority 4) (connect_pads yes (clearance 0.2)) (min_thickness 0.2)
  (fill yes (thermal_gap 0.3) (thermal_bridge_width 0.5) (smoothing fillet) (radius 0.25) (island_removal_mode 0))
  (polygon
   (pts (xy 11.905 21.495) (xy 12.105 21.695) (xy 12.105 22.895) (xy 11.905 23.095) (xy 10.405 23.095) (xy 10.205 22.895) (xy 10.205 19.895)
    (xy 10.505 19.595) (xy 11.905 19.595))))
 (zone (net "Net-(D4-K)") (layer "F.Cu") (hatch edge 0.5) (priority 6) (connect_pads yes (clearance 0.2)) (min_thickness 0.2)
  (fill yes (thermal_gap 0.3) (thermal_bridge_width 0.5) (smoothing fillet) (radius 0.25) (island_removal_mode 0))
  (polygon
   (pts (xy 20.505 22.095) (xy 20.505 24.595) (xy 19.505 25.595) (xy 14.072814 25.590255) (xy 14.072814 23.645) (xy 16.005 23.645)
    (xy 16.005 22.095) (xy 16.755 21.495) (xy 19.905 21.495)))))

